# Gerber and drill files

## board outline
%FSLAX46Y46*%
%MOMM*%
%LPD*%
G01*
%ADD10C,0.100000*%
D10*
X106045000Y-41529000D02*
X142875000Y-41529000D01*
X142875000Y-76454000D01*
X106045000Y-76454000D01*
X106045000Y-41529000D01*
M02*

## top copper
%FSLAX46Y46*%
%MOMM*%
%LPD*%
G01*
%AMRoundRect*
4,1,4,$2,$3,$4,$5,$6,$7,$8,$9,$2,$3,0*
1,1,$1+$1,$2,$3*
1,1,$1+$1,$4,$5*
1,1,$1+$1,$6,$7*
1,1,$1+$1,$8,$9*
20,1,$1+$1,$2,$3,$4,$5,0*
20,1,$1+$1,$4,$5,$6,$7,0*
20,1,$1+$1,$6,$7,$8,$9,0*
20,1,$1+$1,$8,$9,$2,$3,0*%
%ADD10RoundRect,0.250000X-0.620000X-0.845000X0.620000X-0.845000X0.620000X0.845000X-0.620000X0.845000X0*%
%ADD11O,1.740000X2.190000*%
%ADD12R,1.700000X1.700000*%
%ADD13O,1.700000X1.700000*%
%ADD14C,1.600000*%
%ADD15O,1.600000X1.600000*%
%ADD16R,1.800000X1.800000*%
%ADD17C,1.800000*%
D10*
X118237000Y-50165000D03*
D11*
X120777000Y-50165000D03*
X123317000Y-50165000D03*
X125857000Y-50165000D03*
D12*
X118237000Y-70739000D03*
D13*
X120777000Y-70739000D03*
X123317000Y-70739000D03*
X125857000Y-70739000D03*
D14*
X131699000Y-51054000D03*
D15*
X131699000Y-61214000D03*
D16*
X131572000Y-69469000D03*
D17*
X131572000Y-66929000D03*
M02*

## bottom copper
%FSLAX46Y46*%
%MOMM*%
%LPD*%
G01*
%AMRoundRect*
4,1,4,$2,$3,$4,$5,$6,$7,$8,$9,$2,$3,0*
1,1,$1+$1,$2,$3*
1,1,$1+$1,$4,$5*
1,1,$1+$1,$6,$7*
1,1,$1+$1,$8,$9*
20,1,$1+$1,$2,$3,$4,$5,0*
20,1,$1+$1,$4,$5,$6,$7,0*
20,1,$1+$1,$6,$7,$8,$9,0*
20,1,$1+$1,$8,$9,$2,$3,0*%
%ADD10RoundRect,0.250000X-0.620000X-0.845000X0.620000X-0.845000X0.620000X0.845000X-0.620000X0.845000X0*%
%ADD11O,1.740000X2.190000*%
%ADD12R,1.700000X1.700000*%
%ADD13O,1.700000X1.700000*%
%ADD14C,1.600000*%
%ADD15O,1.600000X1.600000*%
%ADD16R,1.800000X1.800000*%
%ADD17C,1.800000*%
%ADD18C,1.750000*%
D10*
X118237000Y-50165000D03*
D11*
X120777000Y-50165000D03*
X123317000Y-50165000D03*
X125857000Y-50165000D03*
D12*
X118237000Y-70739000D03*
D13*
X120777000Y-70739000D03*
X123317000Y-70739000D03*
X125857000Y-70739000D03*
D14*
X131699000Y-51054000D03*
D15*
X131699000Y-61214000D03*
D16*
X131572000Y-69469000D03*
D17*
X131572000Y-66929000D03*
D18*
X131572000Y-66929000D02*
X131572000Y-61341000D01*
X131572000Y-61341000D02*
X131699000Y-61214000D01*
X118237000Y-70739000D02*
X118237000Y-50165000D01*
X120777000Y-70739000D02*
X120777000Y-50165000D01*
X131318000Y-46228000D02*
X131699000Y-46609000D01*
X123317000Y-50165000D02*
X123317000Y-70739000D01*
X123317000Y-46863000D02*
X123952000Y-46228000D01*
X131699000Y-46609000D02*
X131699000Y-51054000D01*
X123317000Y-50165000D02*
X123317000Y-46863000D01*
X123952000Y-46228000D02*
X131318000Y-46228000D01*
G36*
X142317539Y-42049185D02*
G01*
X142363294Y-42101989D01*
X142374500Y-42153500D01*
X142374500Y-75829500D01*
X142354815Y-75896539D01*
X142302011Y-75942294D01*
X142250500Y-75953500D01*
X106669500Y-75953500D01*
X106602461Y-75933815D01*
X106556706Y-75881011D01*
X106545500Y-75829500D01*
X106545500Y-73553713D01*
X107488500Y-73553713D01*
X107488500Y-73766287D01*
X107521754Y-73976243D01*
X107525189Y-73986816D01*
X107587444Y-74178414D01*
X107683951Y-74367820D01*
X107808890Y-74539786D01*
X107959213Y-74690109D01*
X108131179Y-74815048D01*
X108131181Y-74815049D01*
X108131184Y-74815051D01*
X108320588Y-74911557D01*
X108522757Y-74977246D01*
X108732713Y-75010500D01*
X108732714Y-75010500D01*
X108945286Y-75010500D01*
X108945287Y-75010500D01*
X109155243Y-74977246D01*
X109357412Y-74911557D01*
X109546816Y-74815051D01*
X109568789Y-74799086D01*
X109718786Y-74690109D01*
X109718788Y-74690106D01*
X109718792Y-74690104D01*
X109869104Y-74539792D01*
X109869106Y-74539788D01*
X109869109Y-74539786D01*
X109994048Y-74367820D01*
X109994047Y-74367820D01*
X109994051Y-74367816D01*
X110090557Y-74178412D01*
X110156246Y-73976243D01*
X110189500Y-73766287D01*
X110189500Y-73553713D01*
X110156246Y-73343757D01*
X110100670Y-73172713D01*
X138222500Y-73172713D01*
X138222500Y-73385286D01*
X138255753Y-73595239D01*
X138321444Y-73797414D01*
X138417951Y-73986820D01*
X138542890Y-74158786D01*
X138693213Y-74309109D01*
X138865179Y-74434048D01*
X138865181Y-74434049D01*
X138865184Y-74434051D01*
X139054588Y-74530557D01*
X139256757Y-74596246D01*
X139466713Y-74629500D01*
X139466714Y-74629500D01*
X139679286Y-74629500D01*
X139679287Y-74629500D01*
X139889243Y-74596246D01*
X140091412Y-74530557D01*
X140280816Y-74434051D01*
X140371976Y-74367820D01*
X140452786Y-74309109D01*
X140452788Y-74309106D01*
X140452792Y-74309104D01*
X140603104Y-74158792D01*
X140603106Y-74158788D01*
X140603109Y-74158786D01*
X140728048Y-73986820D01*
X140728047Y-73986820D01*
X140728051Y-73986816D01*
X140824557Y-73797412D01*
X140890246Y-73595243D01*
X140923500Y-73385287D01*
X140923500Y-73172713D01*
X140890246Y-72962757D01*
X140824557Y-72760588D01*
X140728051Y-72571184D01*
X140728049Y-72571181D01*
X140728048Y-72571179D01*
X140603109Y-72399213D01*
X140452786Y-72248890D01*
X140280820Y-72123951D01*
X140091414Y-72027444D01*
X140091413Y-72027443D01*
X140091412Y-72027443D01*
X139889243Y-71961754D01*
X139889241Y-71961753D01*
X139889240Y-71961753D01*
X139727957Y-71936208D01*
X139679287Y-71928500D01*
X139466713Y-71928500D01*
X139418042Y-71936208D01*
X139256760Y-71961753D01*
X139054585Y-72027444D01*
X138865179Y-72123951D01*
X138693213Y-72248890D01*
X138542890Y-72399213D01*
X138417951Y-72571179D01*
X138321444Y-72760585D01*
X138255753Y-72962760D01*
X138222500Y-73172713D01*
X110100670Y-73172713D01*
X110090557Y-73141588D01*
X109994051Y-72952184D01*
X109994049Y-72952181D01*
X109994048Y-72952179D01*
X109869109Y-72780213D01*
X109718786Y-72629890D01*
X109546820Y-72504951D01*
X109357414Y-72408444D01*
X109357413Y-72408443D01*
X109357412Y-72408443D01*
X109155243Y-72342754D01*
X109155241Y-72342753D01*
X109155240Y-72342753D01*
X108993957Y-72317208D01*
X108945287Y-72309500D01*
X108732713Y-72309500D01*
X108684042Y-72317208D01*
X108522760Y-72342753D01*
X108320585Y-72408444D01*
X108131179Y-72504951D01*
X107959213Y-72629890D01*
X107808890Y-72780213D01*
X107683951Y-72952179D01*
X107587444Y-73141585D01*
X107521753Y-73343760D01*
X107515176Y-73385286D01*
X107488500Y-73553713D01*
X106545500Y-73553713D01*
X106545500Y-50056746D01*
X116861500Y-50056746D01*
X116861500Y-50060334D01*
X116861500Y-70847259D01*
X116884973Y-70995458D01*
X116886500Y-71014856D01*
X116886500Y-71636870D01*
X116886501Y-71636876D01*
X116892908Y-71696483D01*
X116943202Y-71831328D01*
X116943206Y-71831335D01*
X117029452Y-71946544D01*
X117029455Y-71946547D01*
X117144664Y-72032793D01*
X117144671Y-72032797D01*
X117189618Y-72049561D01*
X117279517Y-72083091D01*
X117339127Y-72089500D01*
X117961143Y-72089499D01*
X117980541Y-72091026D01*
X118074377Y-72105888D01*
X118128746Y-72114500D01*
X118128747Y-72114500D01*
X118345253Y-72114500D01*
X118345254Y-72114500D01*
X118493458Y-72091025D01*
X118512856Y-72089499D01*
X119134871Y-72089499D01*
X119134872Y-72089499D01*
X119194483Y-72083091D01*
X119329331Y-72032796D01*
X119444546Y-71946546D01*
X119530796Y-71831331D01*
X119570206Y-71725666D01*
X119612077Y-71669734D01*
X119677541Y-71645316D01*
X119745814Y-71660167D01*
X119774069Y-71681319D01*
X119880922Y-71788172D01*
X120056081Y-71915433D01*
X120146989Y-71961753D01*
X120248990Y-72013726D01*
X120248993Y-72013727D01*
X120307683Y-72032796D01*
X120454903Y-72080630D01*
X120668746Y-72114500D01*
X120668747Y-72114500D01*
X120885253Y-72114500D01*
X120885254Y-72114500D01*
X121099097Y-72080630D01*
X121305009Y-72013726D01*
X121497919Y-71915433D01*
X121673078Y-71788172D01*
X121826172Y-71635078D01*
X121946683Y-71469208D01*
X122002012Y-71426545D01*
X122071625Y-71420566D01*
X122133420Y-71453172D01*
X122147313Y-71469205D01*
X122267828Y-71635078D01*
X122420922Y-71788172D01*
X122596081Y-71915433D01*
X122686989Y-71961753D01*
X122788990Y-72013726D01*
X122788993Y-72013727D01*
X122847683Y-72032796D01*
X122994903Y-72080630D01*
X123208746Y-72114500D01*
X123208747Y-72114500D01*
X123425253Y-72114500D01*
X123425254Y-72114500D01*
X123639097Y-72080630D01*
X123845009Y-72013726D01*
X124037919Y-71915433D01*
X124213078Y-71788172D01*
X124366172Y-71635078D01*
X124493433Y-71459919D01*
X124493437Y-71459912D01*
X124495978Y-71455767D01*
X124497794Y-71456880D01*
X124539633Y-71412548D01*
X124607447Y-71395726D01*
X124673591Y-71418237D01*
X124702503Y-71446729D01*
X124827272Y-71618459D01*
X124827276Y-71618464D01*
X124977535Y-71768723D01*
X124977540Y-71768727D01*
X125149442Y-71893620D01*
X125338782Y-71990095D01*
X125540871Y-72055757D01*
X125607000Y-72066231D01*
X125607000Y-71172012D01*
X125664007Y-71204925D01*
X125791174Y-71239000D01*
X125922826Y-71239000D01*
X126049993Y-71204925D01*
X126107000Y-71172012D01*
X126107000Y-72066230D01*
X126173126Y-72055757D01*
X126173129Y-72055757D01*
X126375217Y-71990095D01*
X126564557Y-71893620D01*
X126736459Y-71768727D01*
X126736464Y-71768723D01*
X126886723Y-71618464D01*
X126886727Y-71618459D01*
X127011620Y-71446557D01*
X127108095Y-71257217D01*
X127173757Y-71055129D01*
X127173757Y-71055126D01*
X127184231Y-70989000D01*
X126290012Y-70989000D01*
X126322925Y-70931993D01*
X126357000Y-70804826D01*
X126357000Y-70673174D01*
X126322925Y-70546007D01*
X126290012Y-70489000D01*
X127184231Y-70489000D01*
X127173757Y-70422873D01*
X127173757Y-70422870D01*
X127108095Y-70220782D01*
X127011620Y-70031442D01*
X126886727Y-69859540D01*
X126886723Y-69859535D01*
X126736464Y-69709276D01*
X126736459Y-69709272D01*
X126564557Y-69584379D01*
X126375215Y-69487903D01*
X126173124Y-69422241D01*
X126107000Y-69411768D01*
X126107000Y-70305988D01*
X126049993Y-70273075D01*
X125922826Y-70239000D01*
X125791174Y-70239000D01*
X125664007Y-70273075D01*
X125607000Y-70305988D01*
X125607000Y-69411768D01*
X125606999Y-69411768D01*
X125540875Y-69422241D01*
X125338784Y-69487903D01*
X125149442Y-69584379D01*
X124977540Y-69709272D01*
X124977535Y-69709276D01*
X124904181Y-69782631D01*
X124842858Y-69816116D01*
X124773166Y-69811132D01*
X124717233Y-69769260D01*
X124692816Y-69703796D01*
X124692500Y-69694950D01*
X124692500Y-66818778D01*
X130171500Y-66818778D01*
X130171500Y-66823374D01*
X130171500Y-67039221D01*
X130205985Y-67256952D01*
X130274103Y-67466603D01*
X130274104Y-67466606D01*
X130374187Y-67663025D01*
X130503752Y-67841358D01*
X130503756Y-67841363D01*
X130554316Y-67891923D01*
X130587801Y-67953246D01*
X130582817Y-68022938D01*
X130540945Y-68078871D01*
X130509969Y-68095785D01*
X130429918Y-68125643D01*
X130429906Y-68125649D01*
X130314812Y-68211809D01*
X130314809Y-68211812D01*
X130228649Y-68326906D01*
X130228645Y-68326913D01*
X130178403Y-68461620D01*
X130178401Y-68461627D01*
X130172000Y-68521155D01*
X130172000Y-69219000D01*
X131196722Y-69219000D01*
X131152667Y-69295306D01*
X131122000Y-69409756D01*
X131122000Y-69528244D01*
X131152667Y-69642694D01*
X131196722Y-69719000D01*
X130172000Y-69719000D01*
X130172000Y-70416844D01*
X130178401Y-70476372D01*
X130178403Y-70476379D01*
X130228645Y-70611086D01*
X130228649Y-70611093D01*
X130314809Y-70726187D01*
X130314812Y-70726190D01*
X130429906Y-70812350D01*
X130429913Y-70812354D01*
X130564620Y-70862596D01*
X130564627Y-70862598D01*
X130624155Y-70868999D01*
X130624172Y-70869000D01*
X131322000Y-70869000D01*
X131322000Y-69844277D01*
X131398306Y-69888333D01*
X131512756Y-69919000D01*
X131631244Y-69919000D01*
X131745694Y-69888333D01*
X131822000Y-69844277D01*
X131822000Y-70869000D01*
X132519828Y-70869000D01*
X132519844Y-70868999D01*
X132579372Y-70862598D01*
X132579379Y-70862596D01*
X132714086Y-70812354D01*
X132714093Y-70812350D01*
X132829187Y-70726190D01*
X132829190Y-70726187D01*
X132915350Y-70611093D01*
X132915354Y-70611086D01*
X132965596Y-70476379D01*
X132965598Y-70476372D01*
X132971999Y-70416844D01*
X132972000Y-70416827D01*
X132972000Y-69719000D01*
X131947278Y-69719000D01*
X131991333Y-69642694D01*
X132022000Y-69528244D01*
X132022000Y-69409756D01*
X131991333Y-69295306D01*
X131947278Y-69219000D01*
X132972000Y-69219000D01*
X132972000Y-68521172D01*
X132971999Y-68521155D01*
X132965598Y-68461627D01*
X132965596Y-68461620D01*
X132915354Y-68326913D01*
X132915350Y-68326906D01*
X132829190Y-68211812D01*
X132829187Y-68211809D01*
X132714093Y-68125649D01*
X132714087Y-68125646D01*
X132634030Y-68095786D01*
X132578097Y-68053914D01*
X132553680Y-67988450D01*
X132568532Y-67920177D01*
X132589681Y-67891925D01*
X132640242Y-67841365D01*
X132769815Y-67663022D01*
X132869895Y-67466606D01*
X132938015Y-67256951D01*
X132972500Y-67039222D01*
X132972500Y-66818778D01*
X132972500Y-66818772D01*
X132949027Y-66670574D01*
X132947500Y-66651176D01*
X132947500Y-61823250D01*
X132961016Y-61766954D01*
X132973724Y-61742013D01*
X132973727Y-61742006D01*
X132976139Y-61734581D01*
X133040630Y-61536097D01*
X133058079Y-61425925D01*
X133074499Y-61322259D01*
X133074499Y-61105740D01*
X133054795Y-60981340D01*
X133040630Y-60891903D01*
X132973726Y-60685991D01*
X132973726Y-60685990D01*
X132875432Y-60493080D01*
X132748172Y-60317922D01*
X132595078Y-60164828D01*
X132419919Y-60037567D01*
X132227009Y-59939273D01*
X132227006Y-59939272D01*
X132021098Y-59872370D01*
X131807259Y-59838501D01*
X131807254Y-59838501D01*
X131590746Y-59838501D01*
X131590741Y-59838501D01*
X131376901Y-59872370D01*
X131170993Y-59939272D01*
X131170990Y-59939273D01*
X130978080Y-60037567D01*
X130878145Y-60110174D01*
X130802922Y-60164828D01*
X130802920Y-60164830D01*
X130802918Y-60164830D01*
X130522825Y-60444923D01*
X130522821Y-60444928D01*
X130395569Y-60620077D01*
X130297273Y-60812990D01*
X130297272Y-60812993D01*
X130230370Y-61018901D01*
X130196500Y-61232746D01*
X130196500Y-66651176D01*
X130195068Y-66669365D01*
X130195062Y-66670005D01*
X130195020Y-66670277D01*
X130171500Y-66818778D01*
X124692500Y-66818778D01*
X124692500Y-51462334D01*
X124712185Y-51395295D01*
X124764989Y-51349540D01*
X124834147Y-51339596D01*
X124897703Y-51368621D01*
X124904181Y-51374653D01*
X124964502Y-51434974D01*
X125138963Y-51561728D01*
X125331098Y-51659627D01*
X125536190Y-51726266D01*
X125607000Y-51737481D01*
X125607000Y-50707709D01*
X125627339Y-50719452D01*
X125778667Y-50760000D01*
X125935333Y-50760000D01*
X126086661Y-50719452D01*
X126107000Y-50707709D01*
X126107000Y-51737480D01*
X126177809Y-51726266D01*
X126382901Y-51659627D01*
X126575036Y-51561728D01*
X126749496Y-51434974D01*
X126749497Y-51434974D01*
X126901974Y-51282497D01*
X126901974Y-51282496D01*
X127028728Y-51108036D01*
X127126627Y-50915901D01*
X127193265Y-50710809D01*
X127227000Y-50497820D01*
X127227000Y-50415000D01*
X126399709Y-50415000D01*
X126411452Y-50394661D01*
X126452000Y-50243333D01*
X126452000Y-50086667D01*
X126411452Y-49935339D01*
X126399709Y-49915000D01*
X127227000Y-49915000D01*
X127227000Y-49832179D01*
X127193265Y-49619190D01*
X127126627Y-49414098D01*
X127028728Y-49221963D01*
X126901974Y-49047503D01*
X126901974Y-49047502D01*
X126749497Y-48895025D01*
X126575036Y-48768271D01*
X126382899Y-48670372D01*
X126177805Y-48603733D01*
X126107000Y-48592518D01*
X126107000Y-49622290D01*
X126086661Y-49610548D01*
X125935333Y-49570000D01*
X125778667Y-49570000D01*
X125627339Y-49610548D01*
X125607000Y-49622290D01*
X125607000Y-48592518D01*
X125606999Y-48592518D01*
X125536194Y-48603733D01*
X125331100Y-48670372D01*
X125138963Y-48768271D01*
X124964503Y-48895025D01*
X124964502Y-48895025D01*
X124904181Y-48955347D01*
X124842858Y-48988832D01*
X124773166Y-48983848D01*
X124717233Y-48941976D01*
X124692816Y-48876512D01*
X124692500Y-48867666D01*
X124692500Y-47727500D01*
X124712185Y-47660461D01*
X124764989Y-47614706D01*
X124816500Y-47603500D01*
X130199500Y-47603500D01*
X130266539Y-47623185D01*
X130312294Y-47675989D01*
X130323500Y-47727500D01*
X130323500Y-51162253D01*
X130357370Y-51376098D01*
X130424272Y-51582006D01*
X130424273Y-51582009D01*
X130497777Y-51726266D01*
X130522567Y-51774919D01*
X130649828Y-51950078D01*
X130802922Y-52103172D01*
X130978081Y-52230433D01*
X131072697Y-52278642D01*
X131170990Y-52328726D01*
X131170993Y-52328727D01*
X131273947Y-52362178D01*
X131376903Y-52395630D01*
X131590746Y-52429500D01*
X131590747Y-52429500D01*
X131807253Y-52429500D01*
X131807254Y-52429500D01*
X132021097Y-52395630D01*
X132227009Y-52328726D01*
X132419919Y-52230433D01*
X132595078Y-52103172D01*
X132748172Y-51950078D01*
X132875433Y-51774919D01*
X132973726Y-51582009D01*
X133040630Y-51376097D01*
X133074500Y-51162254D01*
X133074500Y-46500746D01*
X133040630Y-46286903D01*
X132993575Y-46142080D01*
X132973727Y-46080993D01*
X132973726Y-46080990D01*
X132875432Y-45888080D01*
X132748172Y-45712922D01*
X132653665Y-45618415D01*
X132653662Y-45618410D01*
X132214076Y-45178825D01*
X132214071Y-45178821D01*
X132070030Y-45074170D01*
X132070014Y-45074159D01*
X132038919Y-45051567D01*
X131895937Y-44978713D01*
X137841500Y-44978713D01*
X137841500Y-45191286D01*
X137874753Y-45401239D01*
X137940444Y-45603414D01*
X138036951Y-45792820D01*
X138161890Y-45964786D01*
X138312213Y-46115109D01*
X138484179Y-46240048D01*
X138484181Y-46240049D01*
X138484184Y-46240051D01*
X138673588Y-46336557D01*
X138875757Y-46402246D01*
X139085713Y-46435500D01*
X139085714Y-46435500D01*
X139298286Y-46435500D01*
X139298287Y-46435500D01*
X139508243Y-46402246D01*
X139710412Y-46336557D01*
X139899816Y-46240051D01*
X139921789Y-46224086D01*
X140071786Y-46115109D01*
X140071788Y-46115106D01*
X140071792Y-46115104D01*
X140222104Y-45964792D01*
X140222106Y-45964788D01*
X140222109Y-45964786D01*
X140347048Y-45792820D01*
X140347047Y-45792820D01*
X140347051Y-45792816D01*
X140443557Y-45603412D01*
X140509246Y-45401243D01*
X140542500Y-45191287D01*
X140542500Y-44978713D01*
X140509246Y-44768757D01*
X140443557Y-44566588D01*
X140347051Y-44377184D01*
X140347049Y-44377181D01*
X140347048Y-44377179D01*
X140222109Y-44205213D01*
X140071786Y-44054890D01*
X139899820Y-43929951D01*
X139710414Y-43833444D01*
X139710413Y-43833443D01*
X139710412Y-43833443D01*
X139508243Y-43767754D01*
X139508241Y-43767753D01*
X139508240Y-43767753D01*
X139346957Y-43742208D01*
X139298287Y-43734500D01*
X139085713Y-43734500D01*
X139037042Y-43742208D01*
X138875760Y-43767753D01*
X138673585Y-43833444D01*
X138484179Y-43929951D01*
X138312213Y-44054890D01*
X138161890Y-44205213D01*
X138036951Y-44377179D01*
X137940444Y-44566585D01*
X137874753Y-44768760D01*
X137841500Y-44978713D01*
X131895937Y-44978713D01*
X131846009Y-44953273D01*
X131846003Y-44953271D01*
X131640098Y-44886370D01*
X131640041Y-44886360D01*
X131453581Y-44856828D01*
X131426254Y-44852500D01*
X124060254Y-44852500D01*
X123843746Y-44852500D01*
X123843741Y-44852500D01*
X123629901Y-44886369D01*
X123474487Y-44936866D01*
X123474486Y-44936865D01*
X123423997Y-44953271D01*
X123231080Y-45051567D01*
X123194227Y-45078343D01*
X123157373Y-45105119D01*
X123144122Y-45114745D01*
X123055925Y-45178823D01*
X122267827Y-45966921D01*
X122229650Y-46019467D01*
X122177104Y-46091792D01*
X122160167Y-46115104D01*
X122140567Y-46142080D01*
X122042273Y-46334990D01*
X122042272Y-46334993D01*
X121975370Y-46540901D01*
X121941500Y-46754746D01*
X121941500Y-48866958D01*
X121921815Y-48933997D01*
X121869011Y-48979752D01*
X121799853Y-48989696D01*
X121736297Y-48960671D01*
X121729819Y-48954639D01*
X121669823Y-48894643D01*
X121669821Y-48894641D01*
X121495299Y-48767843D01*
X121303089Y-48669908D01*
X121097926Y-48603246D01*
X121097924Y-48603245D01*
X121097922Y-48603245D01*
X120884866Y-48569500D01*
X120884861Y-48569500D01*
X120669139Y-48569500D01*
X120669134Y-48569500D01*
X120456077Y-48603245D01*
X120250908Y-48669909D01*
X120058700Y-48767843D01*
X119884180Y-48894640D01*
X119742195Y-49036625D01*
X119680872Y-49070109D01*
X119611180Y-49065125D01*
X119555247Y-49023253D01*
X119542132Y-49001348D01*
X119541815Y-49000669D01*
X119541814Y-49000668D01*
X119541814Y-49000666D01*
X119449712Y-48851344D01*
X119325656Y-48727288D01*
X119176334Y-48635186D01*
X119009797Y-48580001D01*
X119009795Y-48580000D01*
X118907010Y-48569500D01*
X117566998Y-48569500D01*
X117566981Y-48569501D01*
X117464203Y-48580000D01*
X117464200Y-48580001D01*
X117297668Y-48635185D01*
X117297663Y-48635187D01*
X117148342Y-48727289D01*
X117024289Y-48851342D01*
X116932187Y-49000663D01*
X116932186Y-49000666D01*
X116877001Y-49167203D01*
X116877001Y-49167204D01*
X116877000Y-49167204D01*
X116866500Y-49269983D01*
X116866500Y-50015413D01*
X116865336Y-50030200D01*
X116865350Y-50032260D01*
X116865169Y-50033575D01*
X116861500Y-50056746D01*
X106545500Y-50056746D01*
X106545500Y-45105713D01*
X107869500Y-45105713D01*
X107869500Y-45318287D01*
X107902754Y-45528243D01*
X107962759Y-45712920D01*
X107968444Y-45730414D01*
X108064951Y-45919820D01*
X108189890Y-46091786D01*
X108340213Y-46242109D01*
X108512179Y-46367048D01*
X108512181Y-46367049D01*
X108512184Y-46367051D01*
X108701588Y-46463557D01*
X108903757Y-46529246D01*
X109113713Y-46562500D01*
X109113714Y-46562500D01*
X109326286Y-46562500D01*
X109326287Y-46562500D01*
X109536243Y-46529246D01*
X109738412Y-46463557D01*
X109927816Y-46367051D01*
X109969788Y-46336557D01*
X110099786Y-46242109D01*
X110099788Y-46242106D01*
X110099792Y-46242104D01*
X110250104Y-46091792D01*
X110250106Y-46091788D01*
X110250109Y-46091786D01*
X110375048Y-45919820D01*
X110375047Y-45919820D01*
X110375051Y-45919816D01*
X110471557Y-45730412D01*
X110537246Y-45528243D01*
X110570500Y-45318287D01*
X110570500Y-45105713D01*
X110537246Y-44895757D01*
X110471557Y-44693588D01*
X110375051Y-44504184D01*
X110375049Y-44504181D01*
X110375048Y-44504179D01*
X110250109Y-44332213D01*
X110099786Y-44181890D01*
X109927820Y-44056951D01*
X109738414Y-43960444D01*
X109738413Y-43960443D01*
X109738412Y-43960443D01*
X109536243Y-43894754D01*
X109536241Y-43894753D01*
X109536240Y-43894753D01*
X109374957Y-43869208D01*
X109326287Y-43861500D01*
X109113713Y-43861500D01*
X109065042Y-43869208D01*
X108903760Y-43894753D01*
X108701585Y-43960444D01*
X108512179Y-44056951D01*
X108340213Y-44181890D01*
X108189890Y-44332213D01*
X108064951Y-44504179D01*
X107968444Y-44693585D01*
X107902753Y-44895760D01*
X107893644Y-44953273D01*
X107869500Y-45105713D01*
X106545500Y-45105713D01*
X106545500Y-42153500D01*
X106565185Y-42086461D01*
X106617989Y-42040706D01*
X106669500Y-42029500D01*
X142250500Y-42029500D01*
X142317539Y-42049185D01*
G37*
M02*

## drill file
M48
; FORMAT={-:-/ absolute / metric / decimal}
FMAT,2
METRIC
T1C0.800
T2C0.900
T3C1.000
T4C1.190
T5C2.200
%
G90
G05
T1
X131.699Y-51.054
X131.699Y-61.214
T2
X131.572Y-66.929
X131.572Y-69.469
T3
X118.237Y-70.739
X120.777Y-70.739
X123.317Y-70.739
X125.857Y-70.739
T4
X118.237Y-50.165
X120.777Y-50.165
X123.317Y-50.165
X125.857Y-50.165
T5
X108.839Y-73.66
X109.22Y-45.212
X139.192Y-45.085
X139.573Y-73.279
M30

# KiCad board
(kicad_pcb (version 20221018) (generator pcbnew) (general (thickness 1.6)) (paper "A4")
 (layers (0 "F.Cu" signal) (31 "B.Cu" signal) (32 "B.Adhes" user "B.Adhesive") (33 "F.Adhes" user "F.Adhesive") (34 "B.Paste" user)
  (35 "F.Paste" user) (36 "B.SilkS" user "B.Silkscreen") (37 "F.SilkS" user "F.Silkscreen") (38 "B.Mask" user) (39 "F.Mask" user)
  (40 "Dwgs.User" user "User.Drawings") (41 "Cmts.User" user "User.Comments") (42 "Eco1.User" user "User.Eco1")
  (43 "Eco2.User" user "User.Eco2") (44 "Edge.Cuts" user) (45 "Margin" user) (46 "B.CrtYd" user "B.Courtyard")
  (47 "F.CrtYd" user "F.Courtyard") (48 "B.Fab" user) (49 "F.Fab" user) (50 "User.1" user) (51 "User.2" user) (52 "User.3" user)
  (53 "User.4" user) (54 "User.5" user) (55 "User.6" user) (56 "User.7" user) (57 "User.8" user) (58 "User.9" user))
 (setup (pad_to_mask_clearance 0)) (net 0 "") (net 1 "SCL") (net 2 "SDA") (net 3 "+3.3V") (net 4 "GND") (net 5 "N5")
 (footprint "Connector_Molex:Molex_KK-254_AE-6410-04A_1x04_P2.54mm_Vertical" (layer "F.Cu") (at 118.237 50.165)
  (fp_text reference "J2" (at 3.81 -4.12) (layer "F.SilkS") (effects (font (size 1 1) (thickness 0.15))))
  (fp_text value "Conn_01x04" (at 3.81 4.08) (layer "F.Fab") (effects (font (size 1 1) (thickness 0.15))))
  (pad "1" thru_hole roundrect (at 0 0) (size 1.74 2.19) (drill 1.19) (layers "*.Cu" "*.Mask") (roundrect_rratio 0.1436781609) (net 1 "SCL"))
  (pad "2" thru_hole oval (at 2.54 0) (size 1.74 2.19) (drill 1.19) (layers "*.Cu" "*.Mask") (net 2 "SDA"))
  (pad "3" thru_hole oval (at 5.08 0) (size 1.74 2.19) (drill 1.19) (layers "*.Cu" "*.Mask") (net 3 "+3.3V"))
  (pad "4" thru_hole oval (at 7.62 0) (size 1.74 2.19) (drill 1.19) (layers "*.Cu" "*.Mask") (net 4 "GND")))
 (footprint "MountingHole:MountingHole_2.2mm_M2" (layer "F.Cu") (at 139.192 45.085)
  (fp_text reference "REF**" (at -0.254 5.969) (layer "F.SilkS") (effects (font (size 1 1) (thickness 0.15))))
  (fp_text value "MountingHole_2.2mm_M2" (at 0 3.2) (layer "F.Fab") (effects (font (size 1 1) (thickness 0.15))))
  (pad "" np_thru_hole circle (at 0 0) (size 2.2 2.2) (drill 2.2) (layers "*.Cu" "*.Mask")))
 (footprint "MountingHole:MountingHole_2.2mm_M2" (layer "F.Cu") (at 108.839 73.66)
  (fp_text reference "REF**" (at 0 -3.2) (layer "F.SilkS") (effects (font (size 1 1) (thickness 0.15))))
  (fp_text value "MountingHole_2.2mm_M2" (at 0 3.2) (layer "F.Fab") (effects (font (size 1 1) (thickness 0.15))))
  (pad "" np_thru_hole circle (at 0 0) (size 2.2 2.2) (drill 2.2) (layers "*.Cu" "*.Mask")))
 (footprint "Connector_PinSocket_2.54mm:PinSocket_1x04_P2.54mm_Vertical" (layer "F.Cu") (at 118.237 70.739 90)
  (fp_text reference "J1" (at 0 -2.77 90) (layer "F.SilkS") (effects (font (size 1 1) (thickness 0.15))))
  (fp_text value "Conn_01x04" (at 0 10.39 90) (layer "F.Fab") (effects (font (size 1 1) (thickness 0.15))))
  (pad "1" thru_hole rect (at 0 0 90) (size 1.7 1.7) (drill 1) (layers "*.Cu" "*.Mask") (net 1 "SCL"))
  (pad "2" thru_hole oval (at 0 2.54 90) (size 1.7 1.7) (drill 1) (layers "*.Cu" "*.Mask") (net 2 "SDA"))
  (pad "3" thru_hole oval (at 0 5.08 90) (size 1.7 1.7) (drill 1) (layers "*.Cu" "*.Mask") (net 3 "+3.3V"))
  (pad "4" thru_hole oval (at 0 7.62 90) (size 1.7 1.7) (drill 1) (layers "*.Cu" "*.Mask") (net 4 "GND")))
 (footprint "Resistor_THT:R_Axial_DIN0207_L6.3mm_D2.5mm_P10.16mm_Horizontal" (layer "F.Cu") (at 131.699 51.054 -90)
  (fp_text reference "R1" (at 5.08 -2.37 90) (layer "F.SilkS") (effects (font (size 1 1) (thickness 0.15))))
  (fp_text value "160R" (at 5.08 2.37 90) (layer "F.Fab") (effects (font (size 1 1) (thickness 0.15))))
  (pad "1" thru_hole circle (at 0 0 270) (size 1.6 1.6) (drill 0.8) (layers "*.Cu" "*.Mask") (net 3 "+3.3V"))
  (pad "2" thru_hole oval (at 10.16 0 270) (size 1.6 1.6) (drill 0.8) (layers "*.Cu" "*.Mask") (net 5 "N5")))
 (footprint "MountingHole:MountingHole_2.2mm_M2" (layer "F.Cu") (at 109.22 45.212)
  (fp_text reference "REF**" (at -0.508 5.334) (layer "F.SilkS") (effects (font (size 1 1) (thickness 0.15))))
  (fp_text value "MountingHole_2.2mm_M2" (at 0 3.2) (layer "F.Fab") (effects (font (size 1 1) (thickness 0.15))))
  (pad "" np_thru_hole circle (at 0 0) (size 2.2 2.2) (drill 2.2) (layers "*.Cu" "*.Mask")))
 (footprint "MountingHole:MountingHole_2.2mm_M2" (layer "F.Cu") (at 139.573 73.279)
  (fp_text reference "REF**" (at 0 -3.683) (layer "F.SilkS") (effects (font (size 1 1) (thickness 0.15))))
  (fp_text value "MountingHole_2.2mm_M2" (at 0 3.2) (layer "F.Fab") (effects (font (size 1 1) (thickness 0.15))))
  (pad "" np_thru_hole circle (at 0 0) (size 2.2 2.2) (drill 2.2) (layers "*.Cu" "*.Mask")))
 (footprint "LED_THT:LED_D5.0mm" (layer "F.Cu") (at 131.572 69.469 90)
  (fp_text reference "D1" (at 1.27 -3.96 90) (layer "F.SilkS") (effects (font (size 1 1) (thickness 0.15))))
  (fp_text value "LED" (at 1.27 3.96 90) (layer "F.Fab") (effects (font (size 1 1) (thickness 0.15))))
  (pad "1" thru_hole rect (at 0 0 90) (size 1.8 1.8) (drill 0.9) (layers "*.Cu" "*.Mask") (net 4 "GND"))
  (pad "2" thru_hole circle (at 2.54 0 90) (size 1.8 1.8) (drill 0.9) (layers "*.Cu" "*.Mask") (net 5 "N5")))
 (gr_rect (start 106.045 41.529) (end 142.875 76.454) (stroke (width 0.1) (type default)) (fill none) (layer "Edge.Cuts"))
 (segment (start 131.572 66.929) (end 131.572 61.341) (width 1.75) (layer "B.Cu") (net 5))
 (segment (start 131.572 61.341) (end 131.699 61.214) (width 1.75) (layer "B.Cu") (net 5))
 (segment (start 118.237 70.739) (end 118.237 50.165) (width 1.75) (layer "B.Cu") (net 1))
 (segment (start 120.777 70.739) (end 120.777 50.165) (width 1.75) (layer "B.Cu") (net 2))
 (segment (start 131.318 46.228) (end 131.699 46.609) (width 1.75) (layer "B.Cu") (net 3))
 (segment (start 123.317 50.165) (end 123.317 70.739) (width 1.75) (layer "B.Cu") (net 3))
 (segment (start 123.317 46.863) (end 123.952 46.228) (width 1.75) (layer "B.Cu") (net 3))
 (segment (start 131.699 46.609) (end 131.699 51.054) (width 1.75) (layer "B.Cu") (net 3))
 (segment (start 123.317 50.165) (end 123.317 46.863) (width 1.75) (layer "B.Cu") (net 3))
 (segment (start 123.952 46.228) (end 131.318 46.228) (width 1.75) (layer "B.Cu") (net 3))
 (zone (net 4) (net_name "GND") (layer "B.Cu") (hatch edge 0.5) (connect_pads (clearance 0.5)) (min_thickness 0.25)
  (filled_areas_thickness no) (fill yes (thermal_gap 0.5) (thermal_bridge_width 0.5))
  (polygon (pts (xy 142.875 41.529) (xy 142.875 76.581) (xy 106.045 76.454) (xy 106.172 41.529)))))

